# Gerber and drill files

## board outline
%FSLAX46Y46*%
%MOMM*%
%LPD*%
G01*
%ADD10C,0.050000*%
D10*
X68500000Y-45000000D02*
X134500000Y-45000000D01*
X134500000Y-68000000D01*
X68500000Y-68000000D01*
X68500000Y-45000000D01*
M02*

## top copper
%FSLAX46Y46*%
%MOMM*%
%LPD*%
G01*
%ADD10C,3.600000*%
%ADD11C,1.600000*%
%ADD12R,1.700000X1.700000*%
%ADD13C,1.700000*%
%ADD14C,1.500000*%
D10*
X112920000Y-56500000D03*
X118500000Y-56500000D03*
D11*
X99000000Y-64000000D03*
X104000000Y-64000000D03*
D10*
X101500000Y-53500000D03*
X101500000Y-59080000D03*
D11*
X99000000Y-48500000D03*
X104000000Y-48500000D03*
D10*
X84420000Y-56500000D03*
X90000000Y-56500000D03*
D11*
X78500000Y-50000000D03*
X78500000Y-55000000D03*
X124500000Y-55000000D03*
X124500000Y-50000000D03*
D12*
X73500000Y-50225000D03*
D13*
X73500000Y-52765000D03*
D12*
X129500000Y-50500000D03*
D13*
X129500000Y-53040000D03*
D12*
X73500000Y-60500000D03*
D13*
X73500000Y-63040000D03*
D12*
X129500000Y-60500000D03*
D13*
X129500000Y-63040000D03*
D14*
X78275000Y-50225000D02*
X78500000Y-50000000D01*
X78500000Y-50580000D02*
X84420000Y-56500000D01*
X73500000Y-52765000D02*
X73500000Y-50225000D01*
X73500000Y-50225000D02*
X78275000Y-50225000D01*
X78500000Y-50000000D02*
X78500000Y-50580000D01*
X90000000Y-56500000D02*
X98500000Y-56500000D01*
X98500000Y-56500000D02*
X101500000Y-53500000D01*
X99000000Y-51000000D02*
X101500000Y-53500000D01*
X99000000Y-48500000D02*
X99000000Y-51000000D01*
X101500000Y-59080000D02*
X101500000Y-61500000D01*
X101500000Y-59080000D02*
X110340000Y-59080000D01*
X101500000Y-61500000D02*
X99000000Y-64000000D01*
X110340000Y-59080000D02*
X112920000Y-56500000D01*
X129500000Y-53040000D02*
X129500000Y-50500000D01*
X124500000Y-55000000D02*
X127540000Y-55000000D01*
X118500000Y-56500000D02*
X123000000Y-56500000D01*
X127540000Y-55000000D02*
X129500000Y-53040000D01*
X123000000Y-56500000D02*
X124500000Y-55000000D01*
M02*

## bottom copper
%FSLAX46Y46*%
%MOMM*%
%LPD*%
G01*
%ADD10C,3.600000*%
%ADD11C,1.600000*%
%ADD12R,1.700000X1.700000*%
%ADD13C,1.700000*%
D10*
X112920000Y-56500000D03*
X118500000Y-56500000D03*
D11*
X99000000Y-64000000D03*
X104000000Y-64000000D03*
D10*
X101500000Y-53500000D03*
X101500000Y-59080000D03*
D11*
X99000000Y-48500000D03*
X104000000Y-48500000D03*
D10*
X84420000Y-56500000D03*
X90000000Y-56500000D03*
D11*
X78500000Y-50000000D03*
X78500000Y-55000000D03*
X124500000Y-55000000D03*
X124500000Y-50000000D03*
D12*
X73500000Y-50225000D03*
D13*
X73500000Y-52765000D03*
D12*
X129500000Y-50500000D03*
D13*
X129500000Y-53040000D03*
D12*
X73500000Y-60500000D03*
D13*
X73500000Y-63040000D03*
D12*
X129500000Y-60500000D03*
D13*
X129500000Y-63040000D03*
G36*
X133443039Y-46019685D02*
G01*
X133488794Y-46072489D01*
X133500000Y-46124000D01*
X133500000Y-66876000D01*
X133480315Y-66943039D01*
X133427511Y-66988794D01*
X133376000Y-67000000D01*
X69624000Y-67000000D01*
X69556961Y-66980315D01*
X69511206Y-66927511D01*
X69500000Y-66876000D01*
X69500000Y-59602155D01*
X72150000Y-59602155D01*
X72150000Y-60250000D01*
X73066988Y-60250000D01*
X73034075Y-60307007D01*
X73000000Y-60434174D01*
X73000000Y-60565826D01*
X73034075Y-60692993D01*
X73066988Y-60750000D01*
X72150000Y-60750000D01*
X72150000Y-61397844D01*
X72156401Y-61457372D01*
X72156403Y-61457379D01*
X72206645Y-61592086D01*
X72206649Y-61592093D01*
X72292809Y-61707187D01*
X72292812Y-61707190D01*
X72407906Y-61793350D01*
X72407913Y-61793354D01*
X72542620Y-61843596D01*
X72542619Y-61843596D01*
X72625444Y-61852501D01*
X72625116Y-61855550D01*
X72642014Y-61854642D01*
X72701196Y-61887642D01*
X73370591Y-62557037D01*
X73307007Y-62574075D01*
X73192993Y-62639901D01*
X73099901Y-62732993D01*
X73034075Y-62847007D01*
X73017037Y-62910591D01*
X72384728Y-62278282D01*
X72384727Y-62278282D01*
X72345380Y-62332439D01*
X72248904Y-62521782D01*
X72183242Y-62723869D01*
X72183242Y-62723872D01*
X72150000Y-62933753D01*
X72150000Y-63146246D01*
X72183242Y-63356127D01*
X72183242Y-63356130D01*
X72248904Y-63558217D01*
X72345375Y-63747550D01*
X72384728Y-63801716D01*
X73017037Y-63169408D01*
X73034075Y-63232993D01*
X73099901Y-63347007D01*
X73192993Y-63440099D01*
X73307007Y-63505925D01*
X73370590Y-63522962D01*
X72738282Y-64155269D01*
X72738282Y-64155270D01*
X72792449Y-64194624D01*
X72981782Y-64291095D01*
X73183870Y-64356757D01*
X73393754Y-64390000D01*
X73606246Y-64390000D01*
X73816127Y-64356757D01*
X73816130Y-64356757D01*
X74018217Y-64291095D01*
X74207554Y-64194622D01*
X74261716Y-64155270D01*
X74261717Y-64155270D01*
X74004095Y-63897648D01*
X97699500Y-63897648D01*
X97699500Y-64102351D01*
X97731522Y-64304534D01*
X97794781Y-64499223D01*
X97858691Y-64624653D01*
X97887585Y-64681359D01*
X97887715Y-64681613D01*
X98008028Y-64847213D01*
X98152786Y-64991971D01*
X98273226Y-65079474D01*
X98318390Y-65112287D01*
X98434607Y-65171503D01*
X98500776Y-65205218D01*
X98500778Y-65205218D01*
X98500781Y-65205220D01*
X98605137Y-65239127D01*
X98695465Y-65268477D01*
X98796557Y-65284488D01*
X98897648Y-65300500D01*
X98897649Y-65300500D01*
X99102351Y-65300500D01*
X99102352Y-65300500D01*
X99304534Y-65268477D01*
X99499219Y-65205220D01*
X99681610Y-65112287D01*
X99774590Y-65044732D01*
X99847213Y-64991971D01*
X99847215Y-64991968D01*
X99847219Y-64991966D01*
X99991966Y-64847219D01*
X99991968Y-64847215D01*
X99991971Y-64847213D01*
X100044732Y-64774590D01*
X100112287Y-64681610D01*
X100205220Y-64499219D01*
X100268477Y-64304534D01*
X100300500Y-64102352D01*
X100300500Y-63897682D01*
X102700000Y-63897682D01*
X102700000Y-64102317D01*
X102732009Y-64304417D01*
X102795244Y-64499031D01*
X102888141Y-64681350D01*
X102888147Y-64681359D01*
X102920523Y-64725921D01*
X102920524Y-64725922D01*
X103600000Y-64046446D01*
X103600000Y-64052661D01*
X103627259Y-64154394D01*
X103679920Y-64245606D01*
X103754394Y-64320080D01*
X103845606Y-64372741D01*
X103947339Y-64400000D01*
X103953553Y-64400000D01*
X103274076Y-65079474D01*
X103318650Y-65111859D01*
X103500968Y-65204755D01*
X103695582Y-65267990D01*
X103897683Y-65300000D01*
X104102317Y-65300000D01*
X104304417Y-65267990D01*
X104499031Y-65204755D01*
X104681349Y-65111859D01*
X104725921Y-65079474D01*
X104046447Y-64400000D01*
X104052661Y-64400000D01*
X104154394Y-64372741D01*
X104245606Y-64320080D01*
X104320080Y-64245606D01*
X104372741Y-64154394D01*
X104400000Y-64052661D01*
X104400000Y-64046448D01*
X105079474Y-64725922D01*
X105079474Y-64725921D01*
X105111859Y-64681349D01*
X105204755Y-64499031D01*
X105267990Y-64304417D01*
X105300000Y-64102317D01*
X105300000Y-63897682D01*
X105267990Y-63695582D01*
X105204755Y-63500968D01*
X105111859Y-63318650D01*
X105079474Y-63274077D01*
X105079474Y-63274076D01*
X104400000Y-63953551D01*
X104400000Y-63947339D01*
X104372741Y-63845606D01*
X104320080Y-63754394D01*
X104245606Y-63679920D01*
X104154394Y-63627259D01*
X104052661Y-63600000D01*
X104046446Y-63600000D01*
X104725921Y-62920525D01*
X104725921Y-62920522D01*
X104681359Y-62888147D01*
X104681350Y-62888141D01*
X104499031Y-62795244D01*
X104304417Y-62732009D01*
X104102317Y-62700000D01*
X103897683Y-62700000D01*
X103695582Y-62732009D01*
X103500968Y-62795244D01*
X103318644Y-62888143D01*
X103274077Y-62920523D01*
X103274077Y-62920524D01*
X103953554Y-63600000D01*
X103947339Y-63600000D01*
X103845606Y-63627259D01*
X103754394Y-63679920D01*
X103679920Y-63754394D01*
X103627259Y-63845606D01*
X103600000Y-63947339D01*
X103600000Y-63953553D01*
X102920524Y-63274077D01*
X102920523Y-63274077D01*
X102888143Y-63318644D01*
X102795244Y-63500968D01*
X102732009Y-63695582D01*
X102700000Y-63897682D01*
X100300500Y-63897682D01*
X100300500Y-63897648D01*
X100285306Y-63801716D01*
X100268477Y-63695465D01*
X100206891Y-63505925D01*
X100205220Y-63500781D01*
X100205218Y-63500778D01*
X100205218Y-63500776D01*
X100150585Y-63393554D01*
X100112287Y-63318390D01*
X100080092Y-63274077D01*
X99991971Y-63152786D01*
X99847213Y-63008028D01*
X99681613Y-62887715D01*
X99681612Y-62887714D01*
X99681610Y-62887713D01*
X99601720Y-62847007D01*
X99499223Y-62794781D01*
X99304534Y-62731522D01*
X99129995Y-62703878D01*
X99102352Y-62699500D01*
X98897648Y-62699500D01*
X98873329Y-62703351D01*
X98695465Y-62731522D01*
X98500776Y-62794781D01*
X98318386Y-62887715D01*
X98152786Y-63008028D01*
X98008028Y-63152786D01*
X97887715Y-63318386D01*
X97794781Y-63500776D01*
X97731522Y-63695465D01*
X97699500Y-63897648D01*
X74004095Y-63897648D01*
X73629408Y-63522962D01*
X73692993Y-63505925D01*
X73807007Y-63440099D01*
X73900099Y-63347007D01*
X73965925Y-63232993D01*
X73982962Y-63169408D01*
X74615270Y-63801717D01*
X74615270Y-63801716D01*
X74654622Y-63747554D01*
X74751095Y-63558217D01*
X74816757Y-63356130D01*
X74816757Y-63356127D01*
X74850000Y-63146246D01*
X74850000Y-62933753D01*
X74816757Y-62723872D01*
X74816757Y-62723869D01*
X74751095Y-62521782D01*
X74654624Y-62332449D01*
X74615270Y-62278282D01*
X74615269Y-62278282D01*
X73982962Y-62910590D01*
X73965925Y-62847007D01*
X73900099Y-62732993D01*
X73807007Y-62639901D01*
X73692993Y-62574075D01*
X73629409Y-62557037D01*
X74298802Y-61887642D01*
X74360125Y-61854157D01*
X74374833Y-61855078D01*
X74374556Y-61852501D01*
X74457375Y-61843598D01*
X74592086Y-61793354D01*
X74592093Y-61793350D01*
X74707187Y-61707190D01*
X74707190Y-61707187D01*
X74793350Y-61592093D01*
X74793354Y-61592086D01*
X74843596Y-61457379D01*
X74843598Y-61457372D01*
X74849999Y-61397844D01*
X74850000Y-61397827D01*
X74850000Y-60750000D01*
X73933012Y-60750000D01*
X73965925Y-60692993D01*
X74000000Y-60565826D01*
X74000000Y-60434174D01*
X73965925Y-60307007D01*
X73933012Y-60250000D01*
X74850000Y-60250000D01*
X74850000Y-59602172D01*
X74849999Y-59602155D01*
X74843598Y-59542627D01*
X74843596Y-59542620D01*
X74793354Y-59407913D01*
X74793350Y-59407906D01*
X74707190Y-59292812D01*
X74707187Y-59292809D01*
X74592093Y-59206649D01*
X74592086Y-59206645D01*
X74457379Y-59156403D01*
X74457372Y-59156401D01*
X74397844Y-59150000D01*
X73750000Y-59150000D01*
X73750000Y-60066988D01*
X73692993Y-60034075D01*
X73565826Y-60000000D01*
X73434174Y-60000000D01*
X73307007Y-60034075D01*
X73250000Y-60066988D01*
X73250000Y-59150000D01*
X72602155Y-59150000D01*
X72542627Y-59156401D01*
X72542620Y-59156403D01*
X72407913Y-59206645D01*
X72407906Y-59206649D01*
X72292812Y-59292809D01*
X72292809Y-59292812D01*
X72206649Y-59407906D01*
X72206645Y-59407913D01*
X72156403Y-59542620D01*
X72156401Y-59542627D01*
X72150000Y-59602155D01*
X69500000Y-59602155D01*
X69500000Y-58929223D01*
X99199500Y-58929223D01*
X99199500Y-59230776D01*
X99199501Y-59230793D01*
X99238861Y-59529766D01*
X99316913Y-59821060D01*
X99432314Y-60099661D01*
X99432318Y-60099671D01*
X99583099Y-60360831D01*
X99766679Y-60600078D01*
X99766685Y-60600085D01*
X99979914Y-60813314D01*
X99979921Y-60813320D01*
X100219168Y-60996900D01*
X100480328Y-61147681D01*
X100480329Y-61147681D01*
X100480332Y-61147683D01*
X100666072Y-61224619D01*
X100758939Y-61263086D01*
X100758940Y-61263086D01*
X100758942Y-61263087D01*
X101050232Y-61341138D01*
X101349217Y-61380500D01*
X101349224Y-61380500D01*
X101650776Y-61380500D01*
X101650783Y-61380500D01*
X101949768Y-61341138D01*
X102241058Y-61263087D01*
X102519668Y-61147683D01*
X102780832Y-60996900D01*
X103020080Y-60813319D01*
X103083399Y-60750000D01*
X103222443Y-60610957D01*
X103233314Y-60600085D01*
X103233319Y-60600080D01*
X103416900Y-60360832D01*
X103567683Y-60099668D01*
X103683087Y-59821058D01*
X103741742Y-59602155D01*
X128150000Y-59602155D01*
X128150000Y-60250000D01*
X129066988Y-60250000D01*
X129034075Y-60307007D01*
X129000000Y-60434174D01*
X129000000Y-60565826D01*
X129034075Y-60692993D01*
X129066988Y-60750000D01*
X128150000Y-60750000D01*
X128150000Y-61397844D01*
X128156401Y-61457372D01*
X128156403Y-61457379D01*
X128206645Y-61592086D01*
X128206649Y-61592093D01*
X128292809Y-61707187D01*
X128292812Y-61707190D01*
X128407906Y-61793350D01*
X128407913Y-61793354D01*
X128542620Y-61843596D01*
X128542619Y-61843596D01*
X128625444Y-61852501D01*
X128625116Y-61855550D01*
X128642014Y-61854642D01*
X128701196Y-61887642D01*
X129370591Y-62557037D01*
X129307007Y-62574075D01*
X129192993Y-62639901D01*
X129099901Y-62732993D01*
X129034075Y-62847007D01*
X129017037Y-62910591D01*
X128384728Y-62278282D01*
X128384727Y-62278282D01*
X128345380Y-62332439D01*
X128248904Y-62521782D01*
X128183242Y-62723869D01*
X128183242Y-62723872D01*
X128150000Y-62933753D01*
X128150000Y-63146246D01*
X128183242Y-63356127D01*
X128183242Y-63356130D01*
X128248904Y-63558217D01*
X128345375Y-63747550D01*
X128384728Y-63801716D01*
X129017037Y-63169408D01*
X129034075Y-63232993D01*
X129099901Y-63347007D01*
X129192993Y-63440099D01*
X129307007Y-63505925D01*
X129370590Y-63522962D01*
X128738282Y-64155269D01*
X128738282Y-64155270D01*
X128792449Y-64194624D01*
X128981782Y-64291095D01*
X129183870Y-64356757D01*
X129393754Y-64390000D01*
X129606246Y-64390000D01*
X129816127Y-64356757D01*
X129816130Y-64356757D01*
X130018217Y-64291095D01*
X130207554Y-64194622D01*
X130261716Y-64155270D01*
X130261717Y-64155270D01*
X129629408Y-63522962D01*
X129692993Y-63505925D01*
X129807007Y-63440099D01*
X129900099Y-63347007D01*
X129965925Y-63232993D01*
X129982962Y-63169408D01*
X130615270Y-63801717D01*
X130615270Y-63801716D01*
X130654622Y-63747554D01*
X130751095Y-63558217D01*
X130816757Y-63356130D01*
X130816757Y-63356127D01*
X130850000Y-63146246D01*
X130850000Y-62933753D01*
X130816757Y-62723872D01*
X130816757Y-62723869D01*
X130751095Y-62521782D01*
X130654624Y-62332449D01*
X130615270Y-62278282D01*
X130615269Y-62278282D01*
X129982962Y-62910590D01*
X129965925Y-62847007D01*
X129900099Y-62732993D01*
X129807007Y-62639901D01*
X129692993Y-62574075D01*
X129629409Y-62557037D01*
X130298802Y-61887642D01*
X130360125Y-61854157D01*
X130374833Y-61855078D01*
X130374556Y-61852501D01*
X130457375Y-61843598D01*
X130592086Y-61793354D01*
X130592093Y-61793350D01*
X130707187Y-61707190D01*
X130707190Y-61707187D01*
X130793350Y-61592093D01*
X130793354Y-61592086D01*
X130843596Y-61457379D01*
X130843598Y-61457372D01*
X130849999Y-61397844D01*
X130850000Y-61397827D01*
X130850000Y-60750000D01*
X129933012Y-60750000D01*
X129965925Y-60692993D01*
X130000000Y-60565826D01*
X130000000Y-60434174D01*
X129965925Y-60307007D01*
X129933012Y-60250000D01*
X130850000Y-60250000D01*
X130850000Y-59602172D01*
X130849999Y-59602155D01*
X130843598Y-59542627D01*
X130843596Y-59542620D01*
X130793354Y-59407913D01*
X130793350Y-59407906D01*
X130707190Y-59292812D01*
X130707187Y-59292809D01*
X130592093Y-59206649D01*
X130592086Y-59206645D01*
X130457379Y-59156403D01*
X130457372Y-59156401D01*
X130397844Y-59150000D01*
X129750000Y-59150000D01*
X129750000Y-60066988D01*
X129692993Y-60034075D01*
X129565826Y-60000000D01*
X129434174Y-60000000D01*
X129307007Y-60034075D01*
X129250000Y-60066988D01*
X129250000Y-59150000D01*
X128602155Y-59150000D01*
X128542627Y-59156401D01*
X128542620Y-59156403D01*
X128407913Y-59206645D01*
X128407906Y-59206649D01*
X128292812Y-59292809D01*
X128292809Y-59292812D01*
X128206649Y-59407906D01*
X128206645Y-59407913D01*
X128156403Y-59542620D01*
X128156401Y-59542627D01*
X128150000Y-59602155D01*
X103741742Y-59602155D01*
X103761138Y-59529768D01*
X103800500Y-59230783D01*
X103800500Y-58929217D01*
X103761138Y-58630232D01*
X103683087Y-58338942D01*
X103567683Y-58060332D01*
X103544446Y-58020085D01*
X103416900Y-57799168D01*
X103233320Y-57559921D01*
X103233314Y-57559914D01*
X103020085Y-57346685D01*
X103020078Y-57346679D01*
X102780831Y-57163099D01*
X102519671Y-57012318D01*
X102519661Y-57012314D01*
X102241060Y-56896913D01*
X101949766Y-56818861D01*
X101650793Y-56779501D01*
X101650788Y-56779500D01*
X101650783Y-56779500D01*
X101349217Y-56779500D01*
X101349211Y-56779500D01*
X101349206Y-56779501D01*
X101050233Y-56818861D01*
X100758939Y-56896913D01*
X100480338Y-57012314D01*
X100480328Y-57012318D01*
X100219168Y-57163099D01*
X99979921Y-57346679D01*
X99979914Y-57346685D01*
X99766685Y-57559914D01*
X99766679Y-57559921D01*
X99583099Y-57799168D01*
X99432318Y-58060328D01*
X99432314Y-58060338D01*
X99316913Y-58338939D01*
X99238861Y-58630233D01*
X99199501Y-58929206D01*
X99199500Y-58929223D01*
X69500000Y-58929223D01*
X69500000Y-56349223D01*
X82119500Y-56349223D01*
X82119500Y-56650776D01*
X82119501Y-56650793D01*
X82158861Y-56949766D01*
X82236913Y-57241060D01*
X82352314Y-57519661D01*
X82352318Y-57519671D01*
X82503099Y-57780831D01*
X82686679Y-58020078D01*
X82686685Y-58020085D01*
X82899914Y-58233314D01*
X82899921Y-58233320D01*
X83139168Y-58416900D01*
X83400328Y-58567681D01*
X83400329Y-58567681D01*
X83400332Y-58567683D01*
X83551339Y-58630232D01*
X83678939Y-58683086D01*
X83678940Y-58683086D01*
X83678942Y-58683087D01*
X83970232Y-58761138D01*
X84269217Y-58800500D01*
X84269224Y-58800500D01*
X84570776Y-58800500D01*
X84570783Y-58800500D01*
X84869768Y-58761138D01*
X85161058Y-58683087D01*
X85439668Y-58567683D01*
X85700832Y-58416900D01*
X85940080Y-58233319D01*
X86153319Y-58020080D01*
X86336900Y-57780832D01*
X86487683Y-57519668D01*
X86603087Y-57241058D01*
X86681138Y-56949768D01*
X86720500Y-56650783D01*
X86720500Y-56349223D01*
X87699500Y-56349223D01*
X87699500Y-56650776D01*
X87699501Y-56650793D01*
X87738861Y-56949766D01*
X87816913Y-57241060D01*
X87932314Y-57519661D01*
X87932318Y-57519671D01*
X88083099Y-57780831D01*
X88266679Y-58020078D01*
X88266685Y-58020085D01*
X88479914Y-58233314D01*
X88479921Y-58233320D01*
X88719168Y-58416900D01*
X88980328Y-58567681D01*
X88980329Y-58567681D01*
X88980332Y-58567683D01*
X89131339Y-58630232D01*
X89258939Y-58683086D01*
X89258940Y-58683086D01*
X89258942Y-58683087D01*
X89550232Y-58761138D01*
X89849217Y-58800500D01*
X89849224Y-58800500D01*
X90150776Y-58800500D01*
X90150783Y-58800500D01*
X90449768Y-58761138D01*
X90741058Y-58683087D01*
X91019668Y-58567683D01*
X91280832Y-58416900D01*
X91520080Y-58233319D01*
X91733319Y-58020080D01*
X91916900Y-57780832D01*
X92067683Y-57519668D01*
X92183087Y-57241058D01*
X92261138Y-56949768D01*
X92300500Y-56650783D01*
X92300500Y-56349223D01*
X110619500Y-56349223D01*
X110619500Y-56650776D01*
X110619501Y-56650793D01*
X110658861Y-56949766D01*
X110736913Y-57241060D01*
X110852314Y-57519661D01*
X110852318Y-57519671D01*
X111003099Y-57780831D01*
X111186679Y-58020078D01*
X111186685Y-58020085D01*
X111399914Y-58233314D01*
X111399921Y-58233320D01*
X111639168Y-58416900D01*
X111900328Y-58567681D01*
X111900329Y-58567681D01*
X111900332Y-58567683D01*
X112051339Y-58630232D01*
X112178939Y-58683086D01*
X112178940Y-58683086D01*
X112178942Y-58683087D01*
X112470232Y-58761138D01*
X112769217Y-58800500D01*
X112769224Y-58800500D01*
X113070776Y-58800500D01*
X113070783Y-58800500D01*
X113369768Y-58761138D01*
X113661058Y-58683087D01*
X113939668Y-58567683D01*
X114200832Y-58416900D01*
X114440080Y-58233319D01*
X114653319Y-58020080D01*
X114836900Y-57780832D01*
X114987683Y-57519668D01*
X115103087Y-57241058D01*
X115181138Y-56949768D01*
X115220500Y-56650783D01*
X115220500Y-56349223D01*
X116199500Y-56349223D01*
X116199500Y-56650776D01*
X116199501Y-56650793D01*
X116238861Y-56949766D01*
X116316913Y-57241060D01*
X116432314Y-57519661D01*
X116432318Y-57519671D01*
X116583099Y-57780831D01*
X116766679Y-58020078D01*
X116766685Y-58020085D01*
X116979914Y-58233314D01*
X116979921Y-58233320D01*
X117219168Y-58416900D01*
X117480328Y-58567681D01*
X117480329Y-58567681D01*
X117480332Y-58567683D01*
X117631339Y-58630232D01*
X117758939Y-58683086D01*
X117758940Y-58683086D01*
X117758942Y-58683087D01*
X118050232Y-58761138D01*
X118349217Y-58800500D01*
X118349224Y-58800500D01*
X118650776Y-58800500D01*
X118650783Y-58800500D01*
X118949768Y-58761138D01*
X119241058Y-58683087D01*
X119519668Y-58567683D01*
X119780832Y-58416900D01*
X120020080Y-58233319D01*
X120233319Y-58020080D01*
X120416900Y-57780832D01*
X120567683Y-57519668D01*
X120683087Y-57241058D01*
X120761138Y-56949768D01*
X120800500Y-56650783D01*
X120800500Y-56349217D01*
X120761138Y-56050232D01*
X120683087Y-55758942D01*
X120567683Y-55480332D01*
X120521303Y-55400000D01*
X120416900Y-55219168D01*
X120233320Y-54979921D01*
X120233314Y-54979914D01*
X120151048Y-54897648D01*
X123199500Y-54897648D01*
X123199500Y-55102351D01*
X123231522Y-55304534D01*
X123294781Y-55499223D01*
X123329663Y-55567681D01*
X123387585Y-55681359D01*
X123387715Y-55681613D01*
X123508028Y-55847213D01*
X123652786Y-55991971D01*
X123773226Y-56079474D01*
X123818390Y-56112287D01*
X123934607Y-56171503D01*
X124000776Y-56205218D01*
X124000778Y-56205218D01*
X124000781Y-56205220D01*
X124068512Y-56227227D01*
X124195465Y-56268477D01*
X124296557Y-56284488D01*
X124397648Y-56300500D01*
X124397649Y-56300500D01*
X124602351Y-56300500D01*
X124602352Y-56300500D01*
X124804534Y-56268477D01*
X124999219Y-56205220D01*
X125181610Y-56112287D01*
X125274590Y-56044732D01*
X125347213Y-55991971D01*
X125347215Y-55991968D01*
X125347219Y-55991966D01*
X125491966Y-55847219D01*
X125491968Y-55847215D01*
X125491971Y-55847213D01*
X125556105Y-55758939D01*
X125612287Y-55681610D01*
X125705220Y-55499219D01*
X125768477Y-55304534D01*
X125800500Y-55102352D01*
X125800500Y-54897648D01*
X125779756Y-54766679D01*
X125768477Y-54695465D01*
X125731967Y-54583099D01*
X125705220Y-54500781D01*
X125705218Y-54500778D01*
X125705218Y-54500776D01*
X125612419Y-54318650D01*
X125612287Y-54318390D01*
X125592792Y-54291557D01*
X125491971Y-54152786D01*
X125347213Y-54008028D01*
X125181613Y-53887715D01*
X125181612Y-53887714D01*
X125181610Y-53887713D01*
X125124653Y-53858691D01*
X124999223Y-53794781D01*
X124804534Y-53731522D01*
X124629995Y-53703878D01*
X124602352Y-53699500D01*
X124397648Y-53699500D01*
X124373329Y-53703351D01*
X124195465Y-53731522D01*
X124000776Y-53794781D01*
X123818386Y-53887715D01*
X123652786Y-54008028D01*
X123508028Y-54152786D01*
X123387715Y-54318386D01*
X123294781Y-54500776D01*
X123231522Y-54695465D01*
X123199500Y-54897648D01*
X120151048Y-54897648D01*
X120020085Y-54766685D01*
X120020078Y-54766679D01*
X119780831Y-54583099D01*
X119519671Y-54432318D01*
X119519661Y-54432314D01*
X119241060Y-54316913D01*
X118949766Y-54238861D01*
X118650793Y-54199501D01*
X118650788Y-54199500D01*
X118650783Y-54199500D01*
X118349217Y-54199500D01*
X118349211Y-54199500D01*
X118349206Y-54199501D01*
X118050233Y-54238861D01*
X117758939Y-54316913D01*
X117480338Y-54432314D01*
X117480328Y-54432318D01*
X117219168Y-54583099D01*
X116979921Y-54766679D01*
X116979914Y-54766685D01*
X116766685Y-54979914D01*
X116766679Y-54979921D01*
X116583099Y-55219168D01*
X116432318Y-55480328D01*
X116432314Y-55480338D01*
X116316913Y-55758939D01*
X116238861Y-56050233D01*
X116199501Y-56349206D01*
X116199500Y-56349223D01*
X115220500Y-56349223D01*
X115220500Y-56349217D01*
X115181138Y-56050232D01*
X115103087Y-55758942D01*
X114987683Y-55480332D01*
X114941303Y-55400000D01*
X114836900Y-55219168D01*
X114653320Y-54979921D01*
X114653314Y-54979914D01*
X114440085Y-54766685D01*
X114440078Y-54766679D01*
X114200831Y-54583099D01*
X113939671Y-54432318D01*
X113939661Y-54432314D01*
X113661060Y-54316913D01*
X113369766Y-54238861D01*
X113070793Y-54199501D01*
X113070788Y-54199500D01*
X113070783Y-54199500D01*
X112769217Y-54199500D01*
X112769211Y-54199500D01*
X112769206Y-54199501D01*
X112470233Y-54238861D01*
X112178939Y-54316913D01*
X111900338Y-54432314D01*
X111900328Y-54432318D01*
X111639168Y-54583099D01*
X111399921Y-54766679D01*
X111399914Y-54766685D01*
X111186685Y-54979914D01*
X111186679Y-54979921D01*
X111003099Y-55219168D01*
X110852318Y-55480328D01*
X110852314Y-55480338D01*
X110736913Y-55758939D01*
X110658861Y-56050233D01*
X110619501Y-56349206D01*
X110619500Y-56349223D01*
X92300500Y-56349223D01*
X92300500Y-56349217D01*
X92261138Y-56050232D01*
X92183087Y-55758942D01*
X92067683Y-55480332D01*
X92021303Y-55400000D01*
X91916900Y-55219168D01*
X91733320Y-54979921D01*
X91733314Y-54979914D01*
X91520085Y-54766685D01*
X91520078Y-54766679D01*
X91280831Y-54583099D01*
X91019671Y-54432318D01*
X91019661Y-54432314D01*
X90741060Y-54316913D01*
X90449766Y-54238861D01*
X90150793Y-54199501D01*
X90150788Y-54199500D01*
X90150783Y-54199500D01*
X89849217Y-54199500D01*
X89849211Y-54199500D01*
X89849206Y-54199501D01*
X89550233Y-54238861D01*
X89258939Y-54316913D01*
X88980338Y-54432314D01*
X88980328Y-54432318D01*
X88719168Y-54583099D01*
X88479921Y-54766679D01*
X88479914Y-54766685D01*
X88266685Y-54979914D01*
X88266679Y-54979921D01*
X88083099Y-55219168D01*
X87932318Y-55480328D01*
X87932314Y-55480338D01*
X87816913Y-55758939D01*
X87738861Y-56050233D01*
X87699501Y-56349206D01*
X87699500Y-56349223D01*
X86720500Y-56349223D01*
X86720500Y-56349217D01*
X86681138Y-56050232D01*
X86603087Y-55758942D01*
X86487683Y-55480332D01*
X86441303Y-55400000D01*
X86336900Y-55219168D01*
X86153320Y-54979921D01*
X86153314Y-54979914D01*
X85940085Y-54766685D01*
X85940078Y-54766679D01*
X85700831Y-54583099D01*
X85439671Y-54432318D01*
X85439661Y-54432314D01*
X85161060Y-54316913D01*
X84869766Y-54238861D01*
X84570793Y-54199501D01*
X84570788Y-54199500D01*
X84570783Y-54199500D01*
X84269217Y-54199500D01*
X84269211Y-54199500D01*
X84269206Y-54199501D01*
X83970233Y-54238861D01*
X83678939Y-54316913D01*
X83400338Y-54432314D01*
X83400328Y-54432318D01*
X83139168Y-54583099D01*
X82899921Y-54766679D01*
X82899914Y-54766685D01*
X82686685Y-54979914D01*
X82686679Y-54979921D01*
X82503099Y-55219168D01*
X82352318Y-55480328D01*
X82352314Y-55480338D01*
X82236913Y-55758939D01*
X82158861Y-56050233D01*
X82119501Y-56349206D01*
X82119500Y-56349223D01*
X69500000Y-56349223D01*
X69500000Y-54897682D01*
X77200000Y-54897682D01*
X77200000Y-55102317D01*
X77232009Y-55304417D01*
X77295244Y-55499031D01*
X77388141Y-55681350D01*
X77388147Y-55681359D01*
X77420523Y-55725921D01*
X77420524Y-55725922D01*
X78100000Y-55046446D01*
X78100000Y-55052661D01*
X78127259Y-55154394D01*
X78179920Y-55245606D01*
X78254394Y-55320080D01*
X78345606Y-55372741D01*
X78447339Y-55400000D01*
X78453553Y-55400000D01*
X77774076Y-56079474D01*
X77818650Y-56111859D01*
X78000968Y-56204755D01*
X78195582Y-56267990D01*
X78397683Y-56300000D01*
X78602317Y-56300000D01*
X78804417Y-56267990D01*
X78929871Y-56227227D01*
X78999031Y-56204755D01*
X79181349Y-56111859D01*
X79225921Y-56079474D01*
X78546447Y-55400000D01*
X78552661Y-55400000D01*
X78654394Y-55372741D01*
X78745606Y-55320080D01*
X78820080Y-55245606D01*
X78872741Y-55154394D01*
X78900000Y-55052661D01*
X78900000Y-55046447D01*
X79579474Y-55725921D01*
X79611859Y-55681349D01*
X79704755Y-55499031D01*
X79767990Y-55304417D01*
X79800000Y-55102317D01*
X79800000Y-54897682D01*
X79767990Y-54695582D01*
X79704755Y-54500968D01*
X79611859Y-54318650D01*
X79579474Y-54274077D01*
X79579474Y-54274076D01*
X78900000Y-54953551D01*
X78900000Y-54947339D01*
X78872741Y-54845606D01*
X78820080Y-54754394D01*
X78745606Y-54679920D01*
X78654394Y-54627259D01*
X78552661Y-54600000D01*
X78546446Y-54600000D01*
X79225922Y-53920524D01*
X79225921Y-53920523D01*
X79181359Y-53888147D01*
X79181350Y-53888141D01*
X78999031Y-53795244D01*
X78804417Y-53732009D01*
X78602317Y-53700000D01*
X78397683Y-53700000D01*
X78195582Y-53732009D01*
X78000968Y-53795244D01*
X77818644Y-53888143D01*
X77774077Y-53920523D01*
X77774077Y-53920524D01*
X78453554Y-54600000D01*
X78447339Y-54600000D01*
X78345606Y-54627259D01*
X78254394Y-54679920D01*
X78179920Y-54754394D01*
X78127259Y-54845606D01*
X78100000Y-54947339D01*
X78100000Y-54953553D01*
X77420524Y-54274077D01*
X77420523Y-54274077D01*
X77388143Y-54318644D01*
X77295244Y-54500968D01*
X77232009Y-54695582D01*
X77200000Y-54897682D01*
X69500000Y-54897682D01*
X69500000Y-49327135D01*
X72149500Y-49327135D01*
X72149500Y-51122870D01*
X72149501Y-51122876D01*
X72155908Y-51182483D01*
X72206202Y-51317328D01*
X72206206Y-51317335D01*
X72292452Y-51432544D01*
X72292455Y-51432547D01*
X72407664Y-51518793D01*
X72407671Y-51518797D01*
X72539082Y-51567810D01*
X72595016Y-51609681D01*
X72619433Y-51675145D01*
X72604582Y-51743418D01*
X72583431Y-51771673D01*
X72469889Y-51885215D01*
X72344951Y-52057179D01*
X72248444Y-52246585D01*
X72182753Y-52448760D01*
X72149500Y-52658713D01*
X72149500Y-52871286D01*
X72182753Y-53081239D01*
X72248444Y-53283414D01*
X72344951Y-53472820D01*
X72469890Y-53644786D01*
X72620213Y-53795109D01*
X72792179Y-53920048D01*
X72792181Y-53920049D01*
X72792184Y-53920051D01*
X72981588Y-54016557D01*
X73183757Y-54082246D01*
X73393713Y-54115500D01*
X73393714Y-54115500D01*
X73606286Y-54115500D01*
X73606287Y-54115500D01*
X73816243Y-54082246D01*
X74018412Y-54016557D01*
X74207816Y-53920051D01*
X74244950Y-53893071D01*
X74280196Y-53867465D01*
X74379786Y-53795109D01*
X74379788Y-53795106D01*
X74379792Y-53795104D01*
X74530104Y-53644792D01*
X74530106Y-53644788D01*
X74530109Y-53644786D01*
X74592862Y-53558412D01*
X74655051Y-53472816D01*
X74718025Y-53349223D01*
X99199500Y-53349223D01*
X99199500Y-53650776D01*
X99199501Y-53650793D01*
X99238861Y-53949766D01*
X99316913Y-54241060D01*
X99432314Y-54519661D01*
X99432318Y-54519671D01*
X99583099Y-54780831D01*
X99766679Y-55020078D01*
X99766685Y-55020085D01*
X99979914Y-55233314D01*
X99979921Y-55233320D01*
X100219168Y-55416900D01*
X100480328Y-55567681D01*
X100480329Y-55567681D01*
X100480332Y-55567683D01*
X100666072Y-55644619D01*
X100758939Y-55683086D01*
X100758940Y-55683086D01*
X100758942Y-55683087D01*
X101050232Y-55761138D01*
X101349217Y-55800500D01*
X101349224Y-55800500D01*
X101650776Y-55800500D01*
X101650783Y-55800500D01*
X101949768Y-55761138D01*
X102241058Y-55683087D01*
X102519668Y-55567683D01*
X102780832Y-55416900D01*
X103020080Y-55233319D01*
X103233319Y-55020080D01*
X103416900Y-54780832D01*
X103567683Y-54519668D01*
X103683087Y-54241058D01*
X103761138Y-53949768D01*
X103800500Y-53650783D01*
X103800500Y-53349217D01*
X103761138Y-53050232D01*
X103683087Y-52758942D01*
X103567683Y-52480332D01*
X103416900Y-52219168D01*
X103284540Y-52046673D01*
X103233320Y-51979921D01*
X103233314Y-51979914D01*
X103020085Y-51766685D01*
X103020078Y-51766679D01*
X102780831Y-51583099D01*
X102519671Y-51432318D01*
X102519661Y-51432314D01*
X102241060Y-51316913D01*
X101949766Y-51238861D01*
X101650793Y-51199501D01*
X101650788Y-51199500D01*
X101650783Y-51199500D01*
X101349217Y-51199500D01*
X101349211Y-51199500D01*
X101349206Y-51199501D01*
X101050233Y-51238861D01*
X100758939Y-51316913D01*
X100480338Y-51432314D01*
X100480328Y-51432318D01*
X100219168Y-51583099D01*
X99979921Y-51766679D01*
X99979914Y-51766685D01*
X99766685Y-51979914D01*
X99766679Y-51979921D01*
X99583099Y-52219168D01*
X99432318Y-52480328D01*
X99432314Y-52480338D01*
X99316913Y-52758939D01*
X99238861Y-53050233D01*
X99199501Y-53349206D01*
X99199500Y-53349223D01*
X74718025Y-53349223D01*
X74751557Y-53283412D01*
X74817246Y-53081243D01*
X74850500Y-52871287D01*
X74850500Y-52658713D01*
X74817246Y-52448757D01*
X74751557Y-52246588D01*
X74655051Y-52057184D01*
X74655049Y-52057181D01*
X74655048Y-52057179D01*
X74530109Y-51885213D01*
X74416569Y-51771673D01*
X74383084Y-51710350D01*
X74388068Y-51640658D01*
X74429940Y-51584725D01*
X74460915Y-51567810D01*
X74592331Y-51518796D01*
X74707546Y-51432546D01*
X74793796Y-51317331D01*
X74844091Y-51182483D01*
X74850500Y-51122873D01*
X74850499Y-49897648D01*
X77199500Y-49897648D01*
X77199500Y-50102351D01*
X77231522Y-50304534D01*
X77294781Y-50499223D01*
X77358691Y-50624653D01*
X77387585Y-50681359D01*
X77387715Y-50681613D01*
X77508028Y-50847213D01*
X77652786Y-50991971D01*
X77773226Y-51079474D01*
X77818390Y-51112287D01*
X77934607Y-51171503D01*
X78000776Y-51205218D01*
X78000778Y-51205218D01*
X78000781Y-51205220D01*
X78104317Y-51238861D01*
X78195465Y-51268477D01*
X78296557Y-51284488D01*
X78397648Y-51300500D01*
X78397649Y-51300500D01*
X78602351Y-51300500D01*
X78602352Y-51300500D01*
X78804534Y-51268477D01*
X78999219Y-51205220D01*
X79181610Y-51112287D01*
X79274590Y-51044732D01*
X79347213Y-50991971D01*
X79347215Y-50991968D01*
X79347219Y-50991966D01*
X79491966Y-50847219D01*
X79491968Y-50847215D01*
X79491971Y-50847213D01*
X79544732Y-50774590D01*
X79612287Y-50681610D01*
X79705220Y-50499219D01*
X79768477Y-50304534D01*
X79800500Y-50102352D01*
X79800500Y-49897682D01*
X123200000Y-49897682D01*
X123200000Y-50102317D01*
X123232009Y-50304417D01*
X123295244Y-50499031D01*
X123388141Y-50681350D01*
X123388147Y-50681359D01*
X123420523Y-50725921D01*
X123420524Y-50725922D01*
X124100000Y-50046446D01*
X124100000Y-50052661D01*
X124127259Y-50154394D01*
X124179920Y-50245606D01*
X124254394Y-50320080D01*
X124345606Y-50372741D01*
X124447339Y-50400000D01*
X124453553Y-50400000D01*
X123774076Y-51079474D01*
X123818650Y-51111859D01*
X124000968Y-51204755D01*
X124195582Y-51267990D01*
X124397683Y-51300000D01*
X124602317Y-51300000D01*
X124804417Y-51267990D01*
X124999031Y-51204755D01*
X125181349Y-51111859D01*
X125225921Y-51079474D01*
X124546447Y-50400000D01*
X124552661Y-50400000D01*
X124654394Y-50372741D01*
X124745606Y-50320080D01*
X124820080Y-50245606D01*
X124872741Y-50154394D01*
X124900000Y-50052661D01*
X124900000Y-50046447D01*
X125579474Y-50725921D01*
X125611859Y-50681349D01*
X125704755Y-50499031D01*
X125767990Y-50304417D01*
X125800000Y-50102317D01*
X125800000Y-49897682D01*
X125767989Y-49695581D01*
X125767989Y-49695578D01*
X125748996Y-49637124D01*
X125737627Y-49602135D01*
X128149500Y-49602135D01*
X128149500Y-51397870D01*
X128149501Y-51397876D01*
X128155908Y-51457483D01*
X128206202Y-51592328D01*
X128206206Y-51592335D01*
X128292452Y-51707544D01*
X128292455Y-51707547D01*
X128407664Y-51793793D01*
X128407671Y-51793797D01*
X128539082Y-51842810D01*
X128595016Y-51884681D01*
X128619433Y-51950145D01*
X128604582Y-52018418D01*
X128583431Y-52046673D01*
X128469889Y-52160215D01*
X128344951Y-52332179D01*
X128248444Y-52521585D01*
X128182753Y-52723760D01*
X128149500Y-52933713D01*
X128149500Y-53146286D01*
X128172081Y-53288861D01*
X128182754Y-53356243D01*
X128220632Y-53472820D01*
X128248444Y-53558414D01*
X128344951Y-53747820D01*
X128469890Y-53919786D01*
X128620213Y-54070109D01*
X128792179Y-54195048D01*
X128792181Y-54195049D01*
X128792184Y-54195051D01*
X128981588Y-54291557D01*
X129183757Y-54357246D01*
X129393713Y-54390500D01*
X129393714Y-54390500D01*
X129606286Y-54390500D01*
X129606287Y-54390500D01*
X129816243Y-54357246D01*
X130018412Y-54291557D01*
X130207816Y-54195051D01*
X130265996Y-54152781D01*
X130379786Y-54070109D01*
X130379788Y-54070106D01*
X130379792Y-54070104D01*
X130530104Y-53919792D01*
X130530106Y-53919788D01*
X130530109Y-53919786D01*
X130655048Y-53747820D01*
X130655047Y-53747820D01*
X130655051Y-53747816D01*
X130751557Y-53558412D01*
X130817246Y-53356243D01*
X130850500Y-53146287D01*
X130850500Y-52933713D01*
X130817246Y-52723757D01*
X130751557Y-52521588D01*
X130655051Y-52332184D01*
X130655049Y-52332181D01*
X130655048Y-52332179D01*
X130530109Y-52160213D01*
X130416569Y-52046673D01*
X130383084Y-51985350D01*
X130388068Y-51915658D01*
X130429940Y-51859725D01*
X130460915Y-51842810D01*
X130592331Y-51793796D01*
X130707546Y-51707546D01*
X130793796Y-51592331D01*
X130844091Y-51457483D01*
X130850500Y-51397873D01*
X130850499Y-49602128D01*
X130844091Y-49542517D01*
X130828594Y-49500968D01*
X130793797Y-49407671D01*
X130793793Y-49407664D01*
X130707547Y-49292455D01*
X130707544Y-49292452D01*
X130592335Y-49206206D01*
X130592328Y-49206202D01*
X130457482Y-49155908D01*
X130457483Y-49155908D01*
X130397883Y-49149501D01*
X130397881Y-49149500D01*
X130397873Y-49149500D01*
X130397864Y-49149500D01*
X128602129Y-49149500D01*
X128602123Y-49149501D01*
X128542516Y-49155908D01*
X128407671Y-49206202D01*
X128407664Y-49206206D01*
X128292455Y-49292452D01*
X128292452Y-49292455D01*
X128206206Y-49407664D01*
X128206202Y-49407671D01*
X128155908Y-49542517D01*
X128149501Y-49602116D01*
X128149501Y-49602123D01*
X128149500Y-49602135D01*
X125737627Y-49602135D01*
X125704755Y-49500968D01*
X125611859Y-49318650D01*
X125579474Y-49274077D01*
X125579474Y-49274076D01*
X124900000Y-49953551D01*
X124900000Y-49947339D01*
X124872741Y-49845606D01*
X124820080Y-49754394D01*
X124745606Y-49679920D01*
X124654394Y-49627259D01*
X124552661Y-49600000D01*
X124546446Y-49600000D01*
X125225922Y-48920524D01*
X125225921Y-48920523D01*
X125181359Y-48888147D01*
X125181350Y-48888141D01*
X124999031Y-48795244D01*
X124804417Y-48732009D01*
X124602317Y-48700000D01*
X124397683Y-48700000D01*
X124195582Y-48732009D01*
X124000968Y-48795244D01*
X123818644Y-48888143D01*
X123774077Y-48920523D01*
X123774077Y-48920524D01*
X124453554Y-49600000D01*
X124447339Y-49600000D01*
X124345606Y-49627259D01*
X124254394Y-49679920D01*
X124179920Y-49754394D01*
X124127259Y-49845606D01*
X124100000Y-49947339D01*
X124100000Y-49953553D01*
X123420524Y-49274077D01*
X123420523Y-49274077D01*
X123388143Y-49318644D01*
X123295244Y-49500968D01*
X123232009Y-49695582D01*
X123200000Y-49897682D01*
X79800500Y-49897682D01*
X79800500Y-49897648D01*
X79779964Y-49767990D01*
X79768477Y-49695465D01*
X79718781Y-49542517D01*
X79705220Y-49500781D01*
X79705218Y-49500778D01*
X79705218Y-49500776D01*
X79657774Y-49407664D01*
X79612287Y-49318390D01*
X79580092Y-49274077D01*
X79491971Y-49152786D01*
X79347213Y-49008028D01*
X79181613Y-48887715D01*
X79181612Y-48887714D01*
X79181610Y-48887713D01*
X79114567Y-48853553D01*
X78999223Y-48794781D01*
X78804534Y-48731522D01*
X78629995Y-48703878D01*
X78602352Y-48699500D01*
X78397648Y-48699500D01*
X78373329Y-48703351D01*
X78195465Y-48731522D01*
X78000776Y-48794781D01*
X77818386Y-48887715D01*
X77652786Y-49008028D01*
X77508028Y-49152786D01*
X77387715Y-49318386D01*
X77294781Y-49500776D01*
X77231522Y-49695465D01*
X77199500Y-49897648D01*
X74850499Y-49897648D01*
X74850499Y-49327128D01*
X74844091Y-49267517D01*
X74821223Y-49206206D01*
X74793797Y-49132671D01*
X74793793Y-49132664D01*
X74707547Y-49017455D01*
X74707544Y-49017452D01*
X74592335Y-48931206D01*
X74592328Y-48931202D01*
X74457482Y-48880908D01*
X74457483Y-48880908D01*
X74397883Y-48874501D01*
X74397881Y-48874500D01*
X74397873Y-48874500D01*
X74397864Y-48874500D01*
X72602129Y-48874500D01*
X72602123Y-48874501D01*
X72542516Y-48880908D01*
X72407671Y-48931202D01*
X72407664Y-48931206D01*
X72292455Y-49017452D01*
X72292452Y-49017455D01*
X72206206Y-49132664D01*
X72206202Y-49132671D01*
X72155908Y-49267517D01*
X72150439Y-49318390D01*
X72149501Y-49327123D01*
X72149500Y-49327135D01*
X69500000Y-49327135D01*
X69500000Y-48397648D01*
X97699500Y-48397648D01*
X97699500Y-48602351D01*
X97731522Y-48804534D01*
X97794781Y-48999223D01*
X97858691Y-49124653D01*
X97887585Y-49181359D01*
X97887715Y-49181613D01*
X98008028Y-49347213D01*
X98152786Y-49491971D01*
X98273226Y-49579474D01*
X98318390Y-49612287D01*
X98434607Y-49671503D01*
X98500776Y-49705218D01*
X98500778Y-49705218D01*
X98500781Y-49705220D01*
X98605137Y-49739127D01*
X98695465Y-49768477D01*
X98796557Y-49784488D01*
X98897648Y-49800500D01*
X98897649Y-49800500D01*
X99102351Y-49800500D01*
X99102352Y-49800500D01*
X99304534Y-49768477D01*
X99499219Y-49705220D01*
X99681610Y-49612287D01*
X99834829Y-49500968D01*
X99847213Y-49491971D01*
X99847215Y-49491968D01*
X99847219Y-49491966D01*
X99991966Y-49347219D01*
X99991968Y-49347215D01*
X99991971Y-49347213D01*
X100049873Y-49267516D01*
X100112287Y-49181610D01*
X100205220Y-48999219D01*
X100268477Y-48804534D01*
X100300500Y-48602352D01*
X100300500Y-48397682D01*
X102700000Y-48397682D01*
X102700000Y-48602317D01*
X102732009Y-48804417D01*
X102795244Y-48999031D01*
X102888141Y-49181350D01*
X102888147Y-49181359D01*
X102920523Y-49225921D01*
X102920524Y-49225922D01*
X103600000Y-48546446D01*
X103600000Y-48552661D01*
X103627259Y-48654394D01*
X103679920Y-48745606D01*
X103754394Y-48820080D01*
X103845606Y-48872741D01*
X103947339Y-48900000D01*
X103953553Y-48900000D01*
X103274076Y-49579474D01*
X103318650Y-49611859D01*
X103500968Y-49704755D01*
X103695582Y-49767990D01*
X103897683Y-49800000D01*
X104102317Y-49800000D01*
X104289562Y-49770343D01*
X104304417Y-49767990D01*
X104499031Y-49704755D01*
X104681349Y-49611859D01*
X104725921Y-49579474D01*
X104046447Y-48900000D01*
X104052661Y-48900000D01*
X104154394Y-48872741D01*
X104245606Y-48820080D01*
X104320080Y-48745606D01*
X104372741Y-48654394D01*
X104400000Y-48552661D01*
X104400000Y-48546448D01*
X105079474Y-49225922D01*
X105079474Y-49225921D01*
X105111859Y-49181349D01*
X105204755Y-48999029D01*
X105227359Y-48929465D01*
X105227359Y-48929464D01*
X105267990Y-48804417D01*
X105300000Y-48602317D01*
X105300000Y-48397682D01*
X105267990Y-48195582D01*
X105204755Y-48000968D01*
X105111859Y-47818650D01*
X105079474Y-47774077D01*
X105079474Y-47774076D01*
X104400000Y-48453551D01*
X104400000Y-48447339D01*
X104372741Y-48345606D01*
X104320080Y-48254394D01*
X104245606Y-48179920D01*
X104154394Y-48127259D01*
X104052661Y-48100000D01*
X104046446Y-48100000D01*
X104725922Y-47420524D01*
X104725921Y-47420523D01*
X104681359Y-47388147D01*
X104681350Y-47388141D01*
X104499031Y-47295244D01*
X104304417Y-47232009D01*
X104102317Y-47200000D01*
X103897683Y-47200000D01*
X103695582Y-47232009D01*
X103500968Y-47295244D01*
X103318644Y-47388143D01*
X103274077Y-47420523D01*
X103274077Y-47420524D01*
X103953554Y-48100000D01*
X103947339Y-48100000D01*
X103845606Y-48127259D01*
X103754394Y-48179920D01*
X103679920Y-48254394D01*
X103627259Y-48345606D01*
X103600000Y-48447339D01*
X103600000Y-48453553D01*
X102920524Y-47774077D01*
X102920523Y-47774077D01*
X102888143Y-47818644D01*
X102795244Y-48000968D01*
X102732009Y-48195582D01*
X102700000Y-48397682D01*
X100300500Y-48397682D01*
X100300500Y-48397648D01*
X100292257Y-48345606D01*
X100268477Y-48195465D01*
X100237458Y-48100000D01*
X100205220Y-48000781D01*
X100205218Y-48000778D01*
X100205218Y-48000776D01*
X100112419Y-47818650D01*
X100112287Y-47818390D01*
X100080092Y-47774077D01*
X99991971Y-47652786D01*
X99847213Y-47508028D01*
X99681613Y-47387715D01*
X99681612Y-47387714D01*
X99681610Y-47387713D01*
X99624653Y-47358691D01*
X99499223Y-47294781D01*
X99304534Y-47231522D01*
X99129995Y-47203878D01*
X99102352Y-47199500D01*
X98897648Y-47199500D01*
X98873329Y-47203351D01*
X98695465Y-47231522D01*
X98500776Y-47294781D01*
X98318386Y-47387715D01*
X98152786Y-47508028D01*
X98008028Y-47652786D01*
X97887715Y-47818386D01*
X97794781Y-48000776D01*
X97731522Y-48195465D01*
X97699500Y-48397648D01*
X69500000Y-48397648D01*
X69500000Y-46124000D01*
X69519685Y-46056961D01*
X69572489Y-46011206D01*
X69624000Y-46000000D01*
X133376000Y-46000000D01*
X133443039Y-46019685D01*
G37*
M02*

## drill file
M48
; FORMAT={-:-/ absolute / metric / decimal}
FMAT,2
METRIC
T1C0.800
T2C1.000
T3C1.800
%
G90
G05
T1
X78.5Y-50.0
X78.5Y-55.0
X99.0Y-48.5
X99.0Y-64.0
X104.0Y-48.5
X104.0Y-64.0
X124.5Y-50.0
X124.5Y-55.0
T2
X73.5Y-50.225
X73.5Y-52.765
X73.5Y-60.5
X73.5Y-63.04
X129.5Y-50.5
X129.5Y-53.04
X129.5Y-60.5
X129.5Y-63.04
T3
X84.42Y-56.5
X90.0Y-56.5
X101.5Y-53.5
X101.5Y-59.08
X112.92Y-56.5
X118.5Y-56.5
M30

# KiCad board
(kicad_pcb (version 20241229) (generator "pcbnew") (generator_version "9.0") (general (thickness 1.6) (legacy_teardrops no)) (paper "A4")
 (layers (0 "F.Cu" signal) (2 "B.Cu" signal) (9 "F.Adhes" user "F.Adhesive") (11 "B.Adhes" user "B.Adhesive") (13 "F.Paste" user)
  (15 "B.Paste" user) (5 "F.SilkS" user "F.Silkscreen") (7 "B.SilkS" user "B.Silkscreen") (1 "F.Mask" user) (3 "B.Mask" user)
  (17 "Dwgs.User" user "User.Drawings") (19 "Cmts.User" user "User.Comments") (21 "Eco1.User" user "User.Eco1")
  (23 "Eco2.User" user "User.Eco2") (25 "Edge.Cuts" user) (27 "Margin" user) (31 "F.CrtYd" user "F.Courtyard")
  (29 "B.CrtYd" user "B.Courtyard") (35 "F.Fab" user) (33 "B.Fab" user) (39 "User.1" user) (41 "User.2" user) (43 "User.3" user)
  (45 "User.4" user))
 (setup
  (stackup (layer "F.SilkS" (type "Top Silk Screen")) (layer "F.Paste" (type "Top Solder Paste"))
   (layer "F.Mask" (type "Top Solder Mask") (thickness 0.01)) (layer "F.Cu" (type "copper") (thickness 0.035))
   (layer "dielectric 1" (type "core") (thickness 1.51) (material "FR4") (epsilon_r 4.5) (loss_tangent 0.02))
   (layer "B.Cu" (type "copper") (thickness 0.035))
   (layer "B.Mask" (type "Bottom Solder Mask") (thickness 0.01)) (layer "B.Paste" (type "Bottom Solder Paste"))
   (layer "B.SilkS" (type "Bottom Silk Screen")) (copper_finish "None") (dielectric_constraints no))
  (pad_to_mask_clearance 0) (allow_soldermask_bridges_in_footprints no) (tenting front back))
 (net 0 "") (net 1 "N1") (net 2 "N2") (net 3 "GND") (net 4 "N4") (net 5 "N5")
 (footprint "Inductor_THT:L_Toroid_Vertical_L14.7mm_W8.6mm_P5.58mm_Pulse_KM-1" (layer "F.Cu") (at 112.92 56.5 90)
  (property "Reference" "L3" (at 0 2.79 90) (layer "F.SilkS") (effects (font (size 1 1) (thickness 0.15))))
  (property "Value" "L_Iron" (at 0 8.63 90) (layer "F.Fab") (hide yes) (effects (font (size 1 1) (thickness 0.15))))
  (pad "1" thru_hole circle (at 0 0 90) (size 3.6 3.6) (drill 1.8) (layers "*.Cu" "*.Mask") (remove_unused_layers no) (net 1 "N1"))
  (pad "2" thru_hole circle (at 0 5.58 90) (size 3.6 3.6) (drill 1.8) (layers "*.Cu" "*.Mask") (remove_unused_layers no) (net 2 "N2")))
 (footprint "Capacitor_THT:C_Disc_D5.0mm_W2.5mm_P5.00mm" (layer "F.Cu") (at 99 64)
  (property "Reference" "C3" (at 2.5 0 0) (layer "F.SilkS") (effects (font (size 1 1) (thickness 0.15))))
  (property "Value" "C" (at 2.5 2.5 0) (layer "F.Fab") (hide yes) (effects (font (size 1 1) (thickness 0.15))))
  (pad "1" thru_hole circle (at 0 0) (size 1.6 1.6) (drill 0.8) (layers "*.Cu" "*.Mask") (remove_unused_layers no) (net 1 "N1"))
  (pad "2" thru_hole circle (at 5 0) (size 1.6 1.6) (drill 0.8) (layers "*.Cu" "*.Mask") (remove_unused_layers no) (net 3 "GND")))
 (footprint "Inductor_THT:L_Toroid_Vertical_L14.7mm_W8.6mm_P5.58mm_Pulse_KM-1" (layer "F.Cu") (at 101.5 53.5)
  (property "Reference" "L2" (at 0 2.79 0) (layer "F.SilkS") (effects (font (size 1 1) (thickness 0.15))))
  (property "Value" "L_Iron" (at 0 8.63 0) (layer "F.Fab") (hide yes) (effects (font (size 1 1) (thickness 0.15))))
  (pad "1" thru_hole circle (at 0 0) (size 3.6 3.6) (drill 1.8) (layers "*.Cu" "*.Mask") (remove_unused_layers no) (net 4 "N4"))
  (pad "2" thru_hole circle (at 0 5.58) (size 3.6 3.6) (drill 1.8) (layers "*.Cu" "*.Mask") (remove_unused_layers no) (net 1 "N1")))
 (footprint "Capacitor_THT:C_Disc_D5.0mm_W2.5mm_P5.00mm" (layer "F.Cu") (at 99 48.5)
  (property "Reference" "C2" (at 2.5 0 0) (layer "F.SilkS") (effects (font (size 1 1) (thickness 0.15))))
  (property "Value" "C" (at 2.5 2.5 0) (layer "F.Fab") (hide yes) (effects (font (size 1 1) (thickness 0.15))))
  (pad "1" thru_hole circle (at 0 0) (size 1.6 1.6) (drill 0.8) (layers "*.Cu" "*.Mask") (remove_unused_layers no) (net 4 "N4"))
  (pad "2" thru_hole circle (at 5 0) (size 1.6 1.6) (drill 0.8) (layers "*.Cu" "*.Mask") (remove_unused_layers no) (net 3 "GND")))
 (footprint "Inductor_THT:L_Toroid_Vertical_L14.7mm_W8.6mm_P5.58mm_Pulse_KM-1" (layer "F.Cu") (at 84.42 56.5 90)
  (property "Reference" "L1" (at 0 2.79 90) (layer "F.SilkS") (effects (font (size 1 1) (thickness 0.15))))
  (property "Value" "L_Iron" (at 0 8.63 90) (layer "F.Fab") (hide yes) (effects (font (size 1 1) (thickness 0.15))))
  (pad "1" thru_hole circle (at 0 0 90) (size 3.6 3.6) (drill 1.8) (layers "*.Cu" "*.Mask") (remove_unused_layers no) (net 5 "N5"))
  (pad "2" thru_hole circle (at 0 5.58 90) (size 3.6 3.6) (drill 1.8) (layers "*.Cu" "*.Mask") (remove_unused_layers no) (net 4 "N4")))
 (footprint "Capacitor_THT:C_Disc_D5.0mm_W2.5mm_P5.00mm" (layer "F.Cu") (at 78.5 50 -90)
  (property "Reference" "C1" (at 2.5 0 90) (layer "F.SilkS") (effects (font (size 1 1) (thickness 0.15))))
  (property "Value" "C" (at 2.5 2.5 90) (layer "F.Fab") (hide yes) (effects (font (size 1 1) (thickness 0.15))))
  (pad "1" thru_hole circle (at 0 0 270) (size 1.6 1.6) (drill 0.8) (layers "*.Cu" "*.Mask") (remove_unused_layers no) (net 5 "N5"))
  (pad "2" thru_hole circle (at 5 0 270) (size 1.6 1.6) (drill 0.8) (layers "*.Cu" "*.Mask") (remove_unused_layers no) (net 3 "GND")))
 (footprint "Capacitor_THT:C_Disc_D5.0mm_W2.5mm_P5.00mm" (layer "F.Cu") (at 124.5 55 90)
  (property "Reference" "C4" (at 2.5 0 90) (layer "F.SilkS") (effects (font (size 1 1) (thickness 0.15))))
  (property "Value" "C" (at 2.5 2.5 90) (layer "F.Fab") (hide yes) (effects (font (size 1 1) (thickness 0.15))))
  (pad "1" thru_hole circle (at 0 0 90) (size 1.6 1.6) (drill 0.8) (layers "*.Cu" "*.Mask") (remove_unused_layers no) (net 2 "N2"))
  (pad "2" thru_hole circle (at 5 0 90) (size 1.6 1.6) (drill 0.8) (layers "*.Cu" "*.Mask") (remove_unused_layers no) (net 3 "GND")))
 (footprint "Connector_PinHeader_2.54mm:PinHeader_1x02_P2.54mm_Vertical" (layer "B.Cu") (at 73.5 50.225 180)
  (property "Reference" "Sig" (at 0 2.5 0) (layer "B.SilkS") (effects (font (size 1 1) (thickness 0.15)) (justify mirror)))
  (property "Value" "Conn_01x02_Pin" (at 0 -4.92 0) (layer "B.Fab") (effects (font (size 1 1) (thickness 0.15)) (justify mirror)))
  (pad "1" thru_hole rect (at 0 0 180) (size 1.7 1.7) (drill 1) (layers "*.Cu" "*.Mask") (remove_unused_layers no) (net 5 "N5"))
  (pad "2" thru_hole circle (at 0 -2.54 180) (size 1.7 1.7) (drill 1) (layers "*.Cu" "*.Mask") (remove_unused_layers no) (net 5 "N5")))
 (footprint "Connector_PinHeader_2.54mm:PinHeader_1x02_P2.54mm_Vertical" (layer "B.Cu") (at 129.5 50.5 180)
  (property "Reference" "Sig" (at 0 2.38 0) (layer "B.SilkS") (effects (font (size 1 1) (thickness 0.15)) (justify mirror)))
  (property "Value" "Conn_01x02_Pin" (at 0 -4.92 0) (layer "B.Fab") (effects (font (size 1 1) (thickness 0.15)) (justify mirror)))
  (pad "1" thru_hole rect (at 0 0 180) (size 1.7 1.7) (drill 1) (layers "*.Cu" "*.Mask") (remove_unused_layers no) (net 2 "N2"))
  (pad "2" thru_hole circle (at 0 -2.54 180) (size 1.7 1.7) (drill 1) (layers "*.Cu" "*.Mask") (remove_unused_layers no) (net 2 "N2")))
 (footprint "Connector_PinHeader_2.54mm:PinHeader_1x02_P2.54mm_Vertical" (layer "B.Cu") (at 73.5 60.5 180)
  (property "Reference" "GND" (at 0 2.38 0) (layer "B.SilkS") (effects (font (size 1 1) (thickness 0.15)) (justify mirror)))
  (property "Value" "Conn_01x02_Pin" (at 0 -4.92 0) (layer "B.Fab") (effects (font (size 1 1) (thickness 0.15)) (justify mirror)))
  (pad "1" thru_hole rect (at 0 0 180) (size 1.7 1.7) (drill 1) (layers "*.Cu" "*.Mask") (remove_unused_layers no) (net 3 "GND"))
  (pad "2" thru_hole circle (at 0 -2.54 180) (size 1.7 1.7) (drill 1) (layers "*.Cu" "*.Mask") (remove_unused_layers no) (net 3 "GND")))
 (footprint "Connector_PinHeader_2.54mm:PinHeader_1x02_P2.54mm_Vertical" (layer "B.Cu") (at 129.5 60.5 180)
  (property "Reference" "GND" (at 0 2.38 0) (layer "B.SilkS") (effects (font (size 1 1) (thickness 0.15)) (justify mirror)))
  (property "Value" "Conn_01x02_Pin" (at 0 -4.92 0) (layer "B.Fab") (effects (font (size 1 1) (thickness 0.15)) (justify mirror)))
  (pad "1" thru_hole rect (at 0 0 180) (size 1.7 1.7) (drill 1) (layers "*.Cu" "*.Mask") (remove_unused_layers no) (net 3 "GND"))
  (pad "2" thru_hole circle (at 0 -2.54 180) (size 1.7 1.7) (drill 1) (layers "*.Cu" "*.Mask") (remove_unused_layers no) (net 3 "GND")))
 (gr_rect (start 68.5 45) (end 134.5 68) (stroke (width 0.05) (type default)) (fill no) (layer "Edge.Cuts"))
 (segment (start 78.275 50.225) (end 78.5 50) (width 1.5) (layer "F.Cu") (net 5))
 (segment (start 78.5 50.58) (end 84.42 56.5) (width 1.5) (layer "F.Cu") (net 5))
 (segment (start 73.5 52.765) (end 73.5 50.225) (width 1.5) (layer "F.Cu") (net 5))
 (segment (start 73.5 50.225) (end 78.275 50.225) (width 1.5) (layer "F.Cu") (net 5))
 (segment (start 78.5 50) (end 78.5 50.58) (width 1.5) (layer "F.Cu") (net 5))
 (segment (start 90 56.5) (end 98.5 56.5) (width 1.5) (layer "F.Cu") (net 4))
 (segment (start 98.5 56.5) (end 101.5 53.5) (width 1.5) (layer "F.Cu") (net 4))
 (segment (start 99 51) (end 101.5 53.5) (width 1.5) (layer "F.Cu") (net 4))
 (segment (start 99 48.5) (end 99 51) (width 1.5) (layer "F.Cu") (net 4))
 (segment (start 101.5 59.08) (end 101.5 61.5) (width 1.5) (layer "F.Cu") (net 1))
 (segment (start 101.5 59.08) (end 110.34 59.08) (width 1.5) (layer "F.Cu") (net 1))
 (segment (start 101.5 61.5) (end 99 64) (width 1.5) (layer "F.Cu") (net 1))
 (segment (start 110.34 59.08) (end 112.92 56.5) (width 1.5) (layer "F.Cu") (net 1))
 (segment (start 129.5 53.04) (end 129.5 50.5) (width 1.5) (layer "F.Cu") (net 2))
 (segment (start 124.5 55) (end 127.54 55) (width 1.5) (layer "F.Cu") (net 2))
 (segment (start 118.5 56.5) (end 123 56.5) (width 1.5) (layer "F.Cu") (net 2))
 (segment (start 127.54 55) (end 129.5 53.04) (width 1.5) (layer "F.Cu") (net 2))
 (segment (start 123 56.5) (end 124.5 55) (width 1.5) (layer "F.Cu") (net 2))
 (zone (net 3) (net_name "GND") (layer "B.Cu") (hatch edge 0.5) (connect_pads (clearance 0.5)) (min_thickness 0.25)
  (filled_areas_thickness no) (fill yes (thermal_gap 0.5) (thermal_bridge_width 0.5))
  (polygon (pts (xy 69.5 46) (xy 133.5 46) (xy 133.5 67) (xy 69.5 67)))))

